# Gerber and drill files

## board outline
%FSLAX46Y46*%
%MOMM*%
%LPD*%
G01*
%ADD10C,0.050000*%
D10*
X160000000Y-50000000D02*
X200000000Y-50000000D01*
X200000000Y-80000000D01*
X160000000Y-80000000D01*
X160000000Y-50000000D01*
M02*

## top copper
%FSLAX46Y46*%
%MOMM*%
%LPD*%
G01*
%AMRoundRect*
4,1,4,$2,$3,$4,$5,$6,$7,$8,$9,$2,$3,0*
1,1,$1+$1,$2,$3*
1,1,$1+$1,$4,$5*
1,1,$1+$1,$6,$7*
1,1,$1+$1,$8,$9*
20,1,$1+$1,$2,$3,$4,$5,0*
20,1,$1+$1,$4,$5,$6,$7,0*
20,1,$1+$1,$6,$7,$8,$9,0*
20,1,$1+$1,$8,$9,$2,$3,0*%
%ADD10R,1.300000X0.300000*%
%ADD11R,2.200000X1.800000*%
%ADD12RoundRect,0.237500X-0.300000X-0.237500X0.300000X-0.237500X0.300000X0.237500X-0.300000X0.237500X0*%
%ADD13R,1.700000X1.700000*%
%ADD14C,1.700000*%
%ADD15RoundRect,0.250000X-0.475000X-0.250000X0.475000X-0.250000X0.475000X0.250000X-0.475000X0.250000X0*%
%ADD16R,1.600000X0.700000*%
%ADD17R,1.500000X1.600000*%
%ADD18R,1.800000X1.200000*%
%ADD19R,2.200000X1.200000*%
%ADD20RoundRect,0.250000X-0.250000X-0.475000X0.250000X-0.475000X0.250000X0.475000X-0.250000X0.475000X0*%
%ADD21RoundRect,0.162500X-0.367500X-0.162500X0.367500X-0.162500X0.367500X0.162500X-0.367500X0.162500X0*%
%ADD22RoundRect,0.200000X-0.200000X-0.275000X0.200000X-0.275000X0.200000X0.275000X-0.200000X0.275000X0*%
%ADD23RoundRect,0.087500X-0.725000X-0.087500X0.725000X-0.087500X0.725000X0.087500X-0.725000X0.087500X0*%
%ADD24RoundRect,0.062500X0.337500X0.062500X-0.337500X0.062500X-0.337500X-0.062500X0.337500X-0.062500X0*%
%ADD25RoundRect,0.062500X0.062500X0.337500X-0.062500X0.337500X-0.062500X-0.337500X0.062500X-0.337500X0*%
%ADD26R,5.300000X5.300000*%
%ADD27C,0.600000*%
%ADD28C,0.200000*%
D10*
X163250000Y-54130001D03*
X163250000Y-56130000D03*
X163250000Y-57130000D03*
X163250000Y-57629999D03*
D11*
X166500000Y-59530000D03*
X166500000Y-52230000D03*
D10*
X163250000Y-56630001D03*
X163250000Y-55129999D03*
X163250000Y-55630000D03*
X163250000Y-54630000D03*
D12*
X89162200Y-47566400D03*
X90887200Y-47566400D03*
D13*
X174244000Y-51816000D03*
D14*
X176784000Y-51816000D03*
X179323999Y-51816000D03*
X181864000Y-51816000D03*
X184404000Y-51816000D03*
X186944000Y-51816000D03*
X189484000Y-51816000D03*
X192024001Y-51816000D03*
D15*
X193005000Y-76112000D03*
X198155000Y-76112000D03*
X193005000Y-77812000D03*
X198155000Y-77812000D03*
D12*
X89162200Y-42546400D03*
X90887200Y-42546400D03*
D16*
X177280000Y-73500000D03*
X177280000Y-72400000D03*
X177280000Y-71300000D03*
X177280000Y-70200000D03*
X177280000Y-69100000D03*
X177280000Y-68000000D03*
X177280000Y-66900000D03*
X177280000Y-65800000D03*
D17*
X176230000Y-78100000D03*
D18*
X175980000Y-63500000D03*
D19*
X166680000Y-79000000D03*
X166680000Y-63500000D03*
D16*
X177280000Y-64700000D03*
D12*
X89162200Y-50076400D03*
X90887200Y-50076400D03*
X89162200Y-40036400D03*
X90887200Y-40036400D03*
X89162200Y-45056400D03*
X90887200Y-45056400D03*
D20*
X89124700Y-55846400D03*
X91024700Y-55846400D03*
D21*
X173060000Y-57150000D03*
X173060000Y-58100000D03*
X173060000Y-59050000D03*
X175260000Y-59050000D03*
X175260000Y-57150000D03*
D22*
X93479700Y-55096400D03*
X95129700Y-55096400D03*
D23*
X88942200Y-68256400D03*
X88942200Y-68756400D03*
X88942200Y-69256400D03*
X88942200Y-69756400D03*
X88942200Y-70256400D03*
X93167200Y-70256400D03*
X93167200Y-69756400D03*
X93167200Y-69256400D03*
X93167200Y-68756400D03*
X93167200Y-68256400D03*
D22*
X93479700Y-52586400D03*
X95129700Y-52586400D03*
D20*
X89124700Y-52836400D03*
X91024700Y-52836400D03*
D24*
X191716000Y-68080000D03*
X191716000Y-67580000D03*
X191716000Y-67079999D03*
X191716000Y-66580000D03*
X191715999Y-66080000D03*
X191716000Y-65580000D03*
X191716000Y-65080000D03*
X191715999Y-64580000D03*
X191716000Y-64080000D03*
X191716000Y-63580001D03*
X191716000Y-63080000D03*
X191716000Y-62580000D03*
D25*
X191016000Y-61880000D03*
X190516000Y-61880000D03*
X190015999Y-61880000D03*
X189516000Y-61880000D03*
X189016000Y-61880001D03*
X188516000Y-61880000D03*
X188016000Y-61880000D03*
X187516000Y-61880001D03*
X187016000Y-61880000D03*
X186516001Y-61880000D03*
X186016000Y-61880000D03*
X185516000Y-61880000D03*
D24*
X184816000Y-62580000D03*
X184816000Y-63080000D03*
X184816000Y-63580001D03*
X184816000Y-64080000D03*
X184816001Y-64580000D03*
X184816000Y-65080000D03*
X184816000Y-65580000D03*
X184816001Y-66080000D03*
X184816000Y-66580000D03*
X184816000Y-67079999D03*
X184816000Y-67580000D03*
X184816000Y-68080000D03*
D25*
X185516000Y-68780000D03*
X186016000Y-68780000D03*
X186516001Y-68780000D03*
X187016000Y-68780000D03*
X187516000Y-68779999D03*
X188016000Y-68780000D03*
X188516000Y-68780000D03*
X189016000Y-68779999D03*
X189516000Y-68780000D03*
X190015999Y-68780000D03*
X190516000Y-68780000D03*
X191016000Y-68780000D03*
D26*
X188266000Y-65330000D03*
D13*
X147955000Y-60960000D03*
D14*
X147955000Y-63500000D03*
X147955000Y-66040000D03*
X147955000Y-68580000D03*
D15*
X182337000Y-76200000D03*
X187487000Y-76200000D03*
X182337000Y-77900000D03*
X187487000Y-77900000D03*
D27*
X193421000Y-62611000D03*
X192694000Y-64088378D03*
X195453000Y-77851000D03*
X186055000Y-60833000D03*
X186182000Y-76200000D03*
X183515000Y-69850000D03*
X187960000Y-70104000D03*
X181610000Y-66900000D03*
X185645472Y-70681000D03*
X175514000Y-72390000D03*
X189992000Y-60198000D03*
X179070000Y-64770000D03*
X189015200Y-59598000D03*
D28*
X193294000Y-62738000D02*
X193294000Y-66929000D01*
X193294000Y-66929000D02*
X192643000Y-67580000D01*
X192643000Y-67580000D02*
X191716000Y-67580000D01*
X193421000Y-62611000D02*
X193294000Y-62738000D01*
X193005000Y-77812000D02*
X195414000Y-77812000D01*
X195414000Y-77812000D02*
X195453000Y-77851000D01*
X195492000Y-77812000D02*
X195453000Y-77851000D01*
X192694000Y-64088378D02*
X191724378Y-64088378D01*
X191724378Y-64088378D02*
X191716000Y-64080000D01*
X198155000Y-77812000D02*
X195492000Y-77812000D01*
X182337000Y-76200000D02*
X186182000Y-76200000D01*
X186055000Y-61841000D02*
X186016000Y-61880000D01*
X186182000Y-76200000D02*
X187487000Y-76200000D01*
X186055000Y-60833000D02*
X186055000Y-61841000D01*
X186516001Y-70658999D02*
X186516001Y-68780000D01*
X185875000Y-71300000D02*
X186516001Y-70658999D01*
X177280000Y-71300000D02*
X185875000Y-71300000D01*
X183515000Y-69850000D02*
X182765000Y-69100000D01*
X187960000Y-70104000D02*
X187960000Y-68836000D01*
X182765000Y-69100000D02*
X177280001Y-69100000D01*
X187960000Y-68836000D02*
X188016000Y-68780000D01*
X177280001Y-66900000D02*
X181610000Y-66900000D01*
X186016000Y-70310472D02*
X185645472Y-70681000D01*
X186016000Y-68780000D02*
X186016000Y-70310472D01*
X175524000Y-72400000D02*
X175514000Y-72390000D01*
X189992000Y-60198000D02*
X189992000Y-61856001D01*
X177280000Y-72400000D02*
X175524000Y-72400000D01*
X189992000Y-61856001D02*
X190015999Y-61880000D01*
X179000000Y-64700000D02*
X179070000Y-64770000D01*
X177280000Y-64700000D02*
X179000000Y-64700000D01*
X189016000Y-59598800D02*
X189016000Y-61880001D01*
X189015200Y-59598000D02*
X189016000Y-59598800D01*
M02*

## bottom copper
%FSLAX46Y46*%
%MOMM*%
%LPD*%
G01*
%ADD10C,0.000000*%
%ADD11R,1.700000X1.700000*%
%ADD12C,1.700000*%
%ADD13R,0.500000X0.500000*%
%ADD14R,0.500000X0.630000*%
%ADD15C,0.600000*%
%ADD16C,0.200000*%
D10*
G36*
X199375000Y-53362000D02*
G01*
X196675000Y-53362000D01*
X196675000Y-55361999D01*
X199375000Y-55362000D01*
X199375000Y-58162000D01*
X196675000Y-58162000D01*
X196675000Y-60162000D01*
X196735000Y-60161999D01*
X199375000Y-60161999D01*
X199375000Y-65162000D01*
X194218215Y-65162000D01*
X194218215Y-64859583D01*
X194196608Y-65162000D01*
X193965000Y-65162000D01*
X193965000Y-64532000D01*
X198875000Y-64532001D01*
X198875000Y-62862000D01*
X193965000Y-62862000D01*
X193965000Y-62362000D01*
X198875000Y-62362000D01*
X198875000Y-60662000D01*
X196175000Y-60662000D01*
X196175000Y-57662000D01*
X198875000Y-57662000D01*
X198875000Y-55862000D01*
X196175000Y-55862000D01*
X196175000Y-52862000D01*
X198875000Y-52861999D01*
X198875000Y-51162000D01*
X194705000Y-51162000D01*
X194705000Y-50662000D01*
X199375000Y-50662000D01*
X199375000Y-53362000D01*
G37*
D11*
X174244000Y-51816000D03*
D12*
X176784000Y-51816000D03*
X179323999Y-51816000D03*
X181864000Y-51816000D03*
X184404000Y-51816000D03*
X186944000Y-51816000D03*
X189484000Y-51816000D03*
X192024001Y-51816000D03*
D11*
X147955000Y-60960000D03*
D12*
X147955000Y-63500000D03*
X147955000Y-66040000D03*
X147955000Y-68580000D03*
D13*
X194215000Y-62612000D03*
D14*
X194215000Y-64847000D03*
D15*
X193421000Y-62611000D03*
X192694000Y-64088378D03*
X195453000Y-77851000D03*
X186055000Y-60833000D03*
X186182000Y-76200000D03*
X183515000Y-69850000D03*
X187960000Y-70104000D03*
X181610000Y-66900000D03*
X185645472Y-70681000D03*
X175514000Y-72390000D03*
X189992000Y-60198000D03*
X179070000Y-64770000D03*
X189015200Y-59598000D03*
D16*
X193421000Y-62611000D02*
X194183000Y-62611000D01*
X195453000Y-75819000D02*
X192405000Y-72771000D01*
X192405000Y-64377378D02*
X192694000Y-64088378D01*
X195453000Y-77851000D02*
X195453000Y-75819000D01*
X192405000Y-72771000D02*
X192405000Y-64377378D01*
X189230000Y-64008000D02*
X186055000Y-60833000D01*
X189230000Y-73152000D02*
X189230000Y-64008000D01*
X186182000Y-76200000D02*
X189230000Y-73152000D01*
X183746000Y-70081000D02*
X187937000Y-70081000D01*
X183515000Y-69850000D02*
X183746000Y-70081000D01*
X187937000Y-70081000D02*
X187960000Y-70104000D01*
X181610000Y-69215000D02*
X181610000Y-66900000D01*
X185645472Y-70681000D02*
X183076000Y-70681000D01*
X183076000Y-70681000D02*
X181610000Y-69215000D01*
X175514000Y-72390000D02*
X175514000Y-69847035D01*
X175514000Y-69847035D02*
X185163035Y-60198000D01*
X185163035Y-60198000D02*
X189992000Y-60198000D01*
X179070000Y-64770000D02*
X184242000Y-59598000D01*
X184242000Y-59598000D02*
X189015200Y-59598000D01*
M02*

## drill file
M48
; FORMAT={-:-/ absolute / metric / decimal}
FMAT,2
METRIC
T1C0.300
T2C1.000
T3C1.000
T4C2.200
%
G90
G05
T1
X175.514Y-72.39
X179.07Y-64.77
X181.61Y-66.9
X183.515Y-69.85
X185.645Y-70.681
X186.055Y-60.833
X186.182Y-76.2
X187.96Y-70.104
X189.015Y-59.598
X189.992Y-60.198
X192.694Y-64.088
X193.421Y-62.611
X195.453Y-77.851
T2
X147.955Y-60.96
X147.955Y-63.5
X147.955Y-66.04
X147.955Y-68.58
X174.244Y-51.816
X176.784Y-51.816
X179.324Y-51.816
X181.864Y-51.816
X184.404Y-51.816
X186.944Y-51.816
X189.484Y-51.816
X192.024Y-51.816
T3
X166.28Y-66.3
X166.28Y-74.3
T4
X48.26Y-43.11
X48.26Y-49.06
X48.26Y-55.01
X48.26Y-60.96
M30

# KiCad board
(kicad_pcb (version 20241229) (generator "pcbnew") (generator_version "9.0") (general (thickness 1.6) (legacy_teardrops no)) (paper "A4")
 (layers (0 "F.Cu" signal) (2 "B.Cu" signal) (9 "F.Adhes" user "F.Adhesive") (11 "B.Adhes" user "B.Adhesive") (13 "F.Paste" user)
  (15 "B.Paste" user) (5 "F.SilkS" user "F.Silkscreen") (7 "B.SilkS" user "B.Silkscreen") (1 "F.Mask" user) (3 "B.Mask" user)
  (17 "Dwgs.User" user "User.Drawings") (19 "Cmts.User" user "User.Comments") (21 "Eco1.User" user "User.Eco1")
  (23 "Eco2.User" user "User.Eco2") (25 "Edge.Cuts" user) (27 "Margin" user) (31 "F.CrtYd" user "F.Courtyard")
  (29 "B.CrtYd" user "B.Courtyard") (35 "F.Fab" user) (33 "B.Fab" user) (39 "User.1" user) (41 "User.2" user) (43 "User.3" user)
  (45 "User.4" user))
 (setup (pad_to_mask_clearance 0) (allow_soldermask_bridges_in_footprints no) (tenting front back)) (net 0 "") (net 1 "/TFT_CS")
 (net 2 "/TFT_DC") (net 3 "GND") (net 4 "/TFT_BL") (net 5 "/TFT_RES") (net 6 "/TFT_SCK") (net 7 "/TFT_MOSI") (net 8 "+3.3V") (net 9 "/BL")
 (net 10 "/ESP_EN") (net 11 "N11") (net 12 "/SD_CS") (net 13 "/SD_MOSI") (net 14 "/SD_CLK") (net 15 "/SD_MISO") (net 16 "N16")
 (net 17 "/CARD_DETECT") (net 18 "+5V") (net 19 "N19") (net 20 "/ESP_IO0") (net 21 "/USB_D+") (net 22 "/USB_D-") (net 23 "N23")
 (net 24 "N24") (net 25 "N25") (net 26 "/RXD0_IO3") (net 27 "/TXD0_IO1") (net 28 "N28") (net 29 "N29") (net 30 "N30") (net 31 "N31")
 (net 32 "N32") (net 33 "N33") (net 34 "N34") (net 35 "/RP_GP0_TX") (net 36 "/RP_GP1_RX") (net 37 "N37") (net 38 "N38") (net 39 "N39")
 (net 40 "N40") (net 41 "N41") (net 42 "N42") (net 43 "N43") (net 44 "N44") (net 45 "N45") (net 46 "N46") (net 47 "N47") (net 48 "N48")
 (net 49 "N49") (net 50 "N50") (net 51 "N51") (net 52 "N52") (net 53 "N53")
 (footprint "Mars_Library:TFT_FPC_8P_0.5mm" (layer "F.Cu") (at 165.1 55.88 90)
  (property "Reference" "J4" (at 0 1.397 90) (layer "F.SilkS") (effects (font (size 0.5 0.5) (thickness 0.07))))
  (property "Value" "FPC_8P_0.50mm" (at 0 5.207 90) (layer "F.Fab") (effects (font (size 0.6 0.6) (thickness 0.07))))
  (pad "CS" smd rect (at 1.749999 -1.85 90) (size 0.3 1.3) (layers "F.Cu" "F.Mask" "F.Paste") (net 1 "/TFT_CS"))
  (pad "DC" smd rect (at -0.25 -1.85 90) (size 0.3 1.3) (layers "F.Cu" "F.Mask" "F.Paste") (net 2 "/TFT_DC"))
  (pad "GND" smd rect (at -1.25 -1.85 90) (size 0.3 1.3) (layers "F.Cu" "F.Mask" "F.Paste") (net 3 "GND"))
  (pad "LEDA" smd rect (at -1.749999 -1.85 90) (size 0.3 1.3) (layers "F.Cu" "F.Mask" "F.Paste") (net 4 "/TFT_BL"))
  (pad "MP" smd rect (at -3.65 1.4 90) (size 1.8 2.2) (layers "F.Cu" "F.Mask" "F.Paste"))
  (pad "MP" smd rect (at 3.65 1.4 90) (size 1.8 2.2) (layers "F.Cu" "F.Mask" "F.Paste"))
  (pad "RES" smd rect (at -0.750001 -1.85 90) (size 0.3 1.3) (layers "F.Cu" "F.Mask" "F.Paste") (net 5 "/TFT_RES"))
  (pad "SCL" smd rect (at 0.750001 -1.85 90) (size 0.3 1.3) (layers "F.Cu" "F.Mask" "F.Paste") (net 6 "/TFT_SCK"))
  (pad "SDA" smd rect (at 0.25 -1.85 90) (size 0.3 1.3) (layers "F.Cu" "F.Mask" "F.Paste") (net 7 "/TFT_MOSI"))
  (pad "VDD" smd rect (at 1.25 -1.85 90) (size 0.3 1.3) (layers "F.Cu" "F.Mask" "F.Paste") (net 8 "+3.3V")))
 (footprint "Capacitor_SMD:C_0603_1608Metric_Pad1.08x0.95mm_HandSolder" (layer "F.Cu") (at 90.0247 47.5664)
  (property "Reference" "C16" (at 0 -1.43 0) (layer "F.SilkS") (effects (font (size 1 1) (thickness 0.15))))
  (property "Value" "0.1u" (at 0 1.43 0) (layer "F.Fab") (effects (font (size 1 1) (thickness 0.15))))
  (pad "1" smd roundrect (at -0.8625 0) (size 1.075 0.95) (layers "F.Cu" "F.Mask" "F.Paste") (roundrect_rratio 0.25) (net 8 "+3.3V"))
  (pad "2" smd roundrect (at 0.8625 0) (size 1.075 0.95) (layers "F.Cu" "F.Mask" "F.Paste") (roundrect_rratio 0.25) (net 3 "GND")))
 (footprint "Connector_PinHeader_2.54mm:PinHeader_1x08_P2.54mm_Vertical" (layer "F.Cu") (at 174.244 51.816 90)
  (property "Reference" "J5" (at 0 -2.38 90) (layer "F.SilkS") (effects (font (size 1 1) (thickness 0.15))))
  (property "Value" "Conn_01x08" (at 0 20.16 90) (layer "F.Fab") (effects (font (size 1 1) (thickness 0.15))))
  (pad "1" thru_hole rect (at 0 0 90) (size 1.7 1.7) (drill 1) (layers "*.Cu" "*.Mask") (remove_unused_layers no) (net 3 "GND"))
  (pad "2" thru_hole circle (at 0 2.54 90) (size 1.7 1.7) (drill 1) (layers "*.Cu" "*.Mask") (remove_unused_layers no) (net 8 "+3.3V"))
  (pad "3" thru_hole circle (at 0 5.079999 90) (size 1.7 1.7) (drill 1) (layers "*.Cu" "*.Mask") (remove_unused_layers no)
   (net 6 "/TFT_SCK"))
  (pad "4" thru_hole circle (at 0 7.62 90) (size 1.7 1.7) (drill 1) (layers "*.Cu" "*.Mask") (remove_unused_layers no) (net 7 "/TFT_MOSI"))
  (pad "5" thru_hole circle (at 0 10.16 90) (size 1.7 1.7) (drill 1) (layers "*.Cu" "*.Mask") (remove_unused_layers no) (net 5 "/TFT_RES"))
  (pad "6" thru_hole circle (at 0 12.7 90) (size 1.7 1.7) (drill 1) (layers "*.Cu" "*.Mask") (remove_unused_layers no) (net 2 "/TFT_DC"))
  (pad "7" thru_hole circle (at 0 15.24 90) (size 1.7 1.7) (drill 1) (layers "*.Cu" "*.Mask") (remove_unused_layers no) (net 1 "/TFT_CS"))
  (pad "8" thru_hole circle (at 0 17.780001 90) (size 1.7 1.7) (drill 1) (layers "*.Cu" "*.Mask") (remove_unused_layers no) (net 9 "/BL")))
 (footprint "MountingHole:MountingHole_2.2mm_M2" (layer "F.Cu") (at 48.26 49.06)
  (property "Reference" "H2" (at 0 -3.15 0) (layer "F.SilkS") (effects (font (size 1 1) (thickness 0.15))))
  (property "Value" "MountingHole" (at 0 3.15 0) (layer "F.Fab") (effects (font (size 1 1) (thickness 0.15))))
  (pad "" np_thru_hole circle (at 0 0) (size 2.2 2.2) (drill 2.2) (layers "*.Cu" "*.Mask")))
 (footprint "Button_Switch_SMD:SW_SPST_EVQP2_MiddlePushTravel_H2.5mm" (layer "F.Cu") (at 195.58 76.962)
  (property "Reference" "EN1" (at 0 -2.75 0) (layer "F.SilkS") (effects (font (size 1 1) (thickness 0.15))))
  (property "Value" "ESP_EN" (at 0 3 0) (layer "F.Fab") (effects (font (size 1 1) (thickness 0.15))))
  (pad "1" smd roundrect (at -2.575 -0.85) (size 1.45 1) (layers "F.Cu" "F.Mask" "F.Paste") (roundrect_rratio 0.25) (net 3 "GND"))
  (pad "1" smd roundrect (at 2.575 -0.85) (size 1.45 1) (layers "F.Cu" "F.Mask" "F.Paste") (roundrect_rratio 0.25) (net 3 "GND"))
  (pad "2" smd roundrect (at -2.575 0.85) (size 1.45 1) (layers "F.Cu" "F.Mask" "F.Paste") (roundrect_rratio 0.25) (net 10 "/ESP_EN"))
  (pad "2" smd roundrect (at 2.575 0.85) (size 1.45 1) (layers "F.Cu" "F.Mask" "F.Paste") (roundrect_rratio 0.25) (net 10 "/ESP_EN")))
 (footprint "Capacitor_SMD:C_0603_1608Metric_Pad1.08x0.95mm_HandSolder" (layer "F.Cu") (at 90.0247 42.5464)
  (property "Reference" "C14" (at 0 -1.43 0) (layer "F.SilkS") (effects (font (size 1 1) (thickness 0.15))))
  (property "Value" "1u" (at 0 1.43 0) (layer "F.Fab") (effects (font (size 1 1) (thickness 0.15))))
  (pad "1" smd roundrect (at -0.8625 0) (size 1.075 0.95) (layers "F.Cu" "F.Mask" "F.Paste") (roundrect_rratio 0.25) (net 8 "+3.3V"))
  (pad "2" smd roundrect (at 0.8625 0) (size 1.075 0.95) (layers "F.Cu" "F.Mask" "F.Paste") (roundrect_rratio 0.25) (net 3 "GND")))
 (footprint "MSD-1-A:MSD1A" (layer "F.Cu") (at 170.18 71.25 -90)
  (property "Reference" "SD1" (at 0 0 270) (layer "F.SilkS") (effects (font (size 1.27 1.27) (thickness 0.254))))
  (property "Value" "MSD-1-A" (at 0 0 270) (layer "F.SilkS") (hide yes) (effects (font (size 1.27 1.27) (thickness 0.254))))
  (pad "" np_thru_hole circle (at -4.95 3.9 270) (size 1 1) (drill 1) (layers "*.Cu" "*.Mask"))
  (pad "" np_thru_hole circle (at 3.05 3.9 270) (size 1 1) (drill 1) (layers "*.Cu" "*.Mask"))
  (pad "1" smd rect (at 2.25 -7.1 270) (size 0.7 1.6) (layers "F.Cu" "F.Mask" "F.Paste") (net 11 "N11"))
  (pad "2" smd rect (at 1.15 -7.1 270) (size 0.7 1.6) (layers "F.Cu" "F.Mask" "F.Paste") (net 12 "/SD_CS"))
  (pad "3" smd rect (at 0.05 -7.1 270) (size 0.7 1.6) (layers "F.Cu" "F.Mask" "F.Paste") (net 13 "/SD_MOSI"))
  (pad "4" smd rect (at -1.05 -7.1 270) (size 0.7 1.6) (layers "F.Cu" "F.Mask" "F.Paste") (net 8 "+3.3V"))
  (pad "5" smd rect (at -2.15 -7.1 270) (size 0.7 1.6) (layers "F.Cu" "F.Mask" "F.Paste") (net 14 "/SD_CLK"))
  (pad "6" smd rect (at -3.25 -7.1 270) (size 0.7 1.6) (layers "F.Cu" "F.Mask" "F.Paste") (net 3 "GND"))
  (pad "7" smd rect (at -4.35 -7.1 270) (size 0.7 1.6) (layers "F.Cu" "F.Mask" "F.Paste") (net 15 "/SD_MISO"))
  (pad "8" smd rect (at -5.45 -7.1 270) (size 0.7 1.6) (layers "F.Cu" "F.Mask" "F.Paste") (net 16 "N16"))
  (pad "9" smd rect (at 6.85 -6.05) (size 1.5 1.6) (layers "F.Cu" "F.Mask" "F.Paste") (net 3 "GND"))
  (pad "10" smd rect (at -7.75 -5.8 270) (size 1.2 1.8) (layers "F.Cu" "F.Mask" "F.Paste") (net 3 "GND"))
  (pad "11" smd rect (at 7.75 3.5 270) (size 1.2 2.2) (layers "F.Cu" "F.Mask" "F.Paste") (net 3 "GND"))
  (pad "12" smd rect (at -7.75 3.5 270) (size 1.2 2.2) (layers "F.Cu" "F.Mask" "F.Paste") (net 3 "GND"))
  (pad "CD1" smd rect (at -6.55 -7.1 270) (size 0.7 1.6) (layers "F.Cu" "F.Mask" "F.Paste") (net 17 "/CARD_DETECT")))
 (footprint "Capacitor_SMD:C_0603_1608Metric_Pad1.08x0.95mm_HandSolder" (layer "F.Cu") (at 90.0247 50.0764)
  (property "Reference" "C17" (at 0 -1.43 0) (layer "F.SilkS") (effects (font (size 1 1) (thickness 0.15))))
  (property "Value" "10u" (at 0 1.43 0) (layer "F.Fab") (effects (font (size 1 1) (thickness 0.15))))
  (pad "1" smd roundrect (at -0.8625 0) (size 1.075 0.95) (layers "F.Cu" "F.Mask" "F.Paste") (roundrect_rratio 0.25) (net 8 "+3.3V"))
  (pad "2" smd roundrect (at 0.8625 0) (size 1.075 0.95) (layers "F.Cu" "F.Mask" "F.Paste") (roundrect_rratio 0.25) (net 3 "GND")))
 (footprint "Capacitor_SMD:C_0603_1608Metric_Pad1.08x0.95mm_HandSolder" (layer "F.Cu") (at 90.0247 40.0364)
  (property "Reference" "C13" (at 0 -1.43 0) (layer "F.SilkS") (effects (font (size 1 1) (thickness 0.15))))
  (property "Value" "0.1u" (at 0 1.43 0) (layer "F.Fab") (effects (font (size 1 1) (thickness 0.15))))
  (pad "1" smd roundrect (at -0.8625 0) (size 1.075 0.95) (layers "F.Cu" "F.Mask" "F.Paste") (roundrect_rratio 0.25) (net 8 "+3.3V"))
  (pad "2" smd roundrect (at 0.8625 0) (size 1.075 0.95) (layers "F.Cu" "F.Mask" "F.Paste") (roundrect_rratio 0.25) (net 3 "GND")))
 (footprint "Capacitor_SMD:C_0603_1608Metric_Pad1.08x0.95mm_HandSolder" (layer "F.Cu") (at 90.0247 45.0564)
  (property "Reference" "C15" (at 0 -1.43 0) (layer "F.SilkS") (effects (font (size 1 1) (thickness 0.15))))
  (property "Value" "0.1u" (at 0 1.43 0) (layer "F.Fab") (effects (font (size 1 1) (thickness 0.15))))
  (pad "1" smd roundrect (at -0.8625 0) (size 1.075 0.95) (layers "F.Cu" "F.Mask" "F.Paste") (roundrect_rratio 0.25) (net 8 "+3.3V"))
  (pad "2" smd roundrect (at 0.8625 0) (size 1.075 0.95) (layers "F.Cu" "F.Mask" "F.Paste") (roundrect_rratio 0.25) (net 3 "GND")))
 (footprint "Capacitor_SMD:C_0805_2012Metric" (layer "F.Cu") (at 90.0747 55.8464)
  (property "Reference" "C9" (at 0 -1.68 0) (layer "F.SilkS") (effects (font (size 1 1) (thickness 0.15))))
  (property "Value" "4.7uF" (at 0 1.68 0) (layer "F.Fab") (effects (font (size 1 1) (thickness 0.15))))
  (pad "1" smd roundrect (at -0.95 0) (size 1 1.45) (layers "F.Cu" "F.Mask" "F.Paste") (roundrect_rratio 0.25) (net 8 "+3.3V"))
  (pad "2" smd roundrect (at 0.95 0) (size 1 1.45) (layers "F.Cu" "F.Mask" "F.Paste") (roundrect_rratio 0.25) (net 3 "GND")))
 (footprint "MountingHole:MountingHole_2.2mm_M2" (layer "F.Cu") (at 48.26 60.96)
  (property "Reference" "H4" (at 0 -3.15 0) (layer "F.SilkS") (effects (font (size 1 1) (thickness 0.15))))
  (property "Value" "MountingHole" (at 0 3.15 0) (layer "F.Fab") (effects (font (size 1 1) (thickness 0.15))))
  (pad "" np_thru_hole circle (at 0 0) (size 2.2 2.2) (drill 2.2) (layers "*.Cu" "*.Mask")))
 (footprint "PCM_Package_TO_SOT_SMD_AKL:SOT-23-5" (layer "F.Cu") (at 174.16 58.1)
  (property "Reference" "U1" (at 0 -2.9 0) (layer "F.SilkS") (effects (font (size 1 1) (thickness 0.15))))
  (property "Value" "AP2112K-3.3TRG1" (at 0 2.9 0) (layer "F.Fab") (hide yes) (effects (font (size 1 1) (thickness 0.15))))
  (pad "1" smd roundrect (at -1.1 -0.95) (size 1.06 0.65) (layers "F.Cu" "F.Mask" "F.Paste") (roundrect_rratio 0.25) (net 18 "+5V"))
  (pad "2" smd roundrect (at -1.1 0) (size 1.06 0.65) (layers "F.Cu" "F.Mask" "F.Paste") (roundrect_rratio 0.25) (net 3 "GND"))
  (pad "3" smd roundrect (at -1.1 0.95) (size 1.06 0.65) (layers "F.Cu" "F.Mask" "F.Paste") (roundrect_rratio 0.25) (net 18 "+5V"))
  (pad "4" smd roundrect (at 1.1 0.95) (size 1.06 0.65) (layers "F.Cu" "F.Mask" "F.Paste") (roundrect_rratio 0.25) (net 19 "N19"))
  (pad "5" smd roundrect (at 1.1 -0.95) (size 1.06 0.65) (layers "F.Cu" "F.Mask" "F.Paste") (roundrect_rratio 0.25) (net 8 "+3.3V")))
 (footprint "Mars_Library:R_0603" (layer "F.Cu") (at 94.3047 55.0964)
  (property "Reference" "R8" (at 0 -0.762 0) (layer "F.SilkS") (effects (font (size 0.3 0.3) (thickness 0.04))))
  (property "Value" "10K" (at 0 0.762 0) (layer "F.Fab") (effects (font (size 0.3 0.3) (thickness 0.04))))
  (pad "1" smd roundrect (at -0.825 0) (size 0.8 0.95) (layers "F.Cu" "F.Mask" "F.Paste") (roundrect_rratio 0.25) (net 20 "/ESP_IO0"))
  (pad "2" smd roundrect (at 0.825 0) (size 0.8 0.95) (layers "F.Cu" "F.Mask" "F.Paste") (roundrect_rratio 0.25) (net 8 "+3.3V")))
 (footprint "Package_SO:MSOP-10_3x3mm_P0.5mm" (layer "F.Cu") (at 91.0547 69.2564)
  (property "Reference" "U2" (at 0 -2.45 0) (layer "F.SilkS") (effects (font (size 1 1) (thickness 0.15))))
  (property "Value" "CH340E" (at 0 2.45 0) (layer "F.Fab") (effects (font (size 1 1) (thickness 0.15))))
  (pad "1" smd roundrect (at -2.1125 -1) (size 1.625 0.35) (layers "F.Cu" "F.Mask" "F.Paste") (roundrect_rratio 0.25) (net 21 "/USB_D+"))
  (pad "2" smd roundrect (at -2.1125 -0.5) (size 1.625 0.35) (layers "F.Cu" "F.Mask" "F.Paste") (roundrect_rratio 0.25) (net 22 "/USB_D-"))
  (pad "3" smd roundrect (at -2.1125 0) (size 1.625 0.35) (layers "F.Cu" "F.Mask" "F.Paste") (roundrect_rratio 0.25) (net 3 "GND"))
  (pad "4" smd roundrect (at -2.1125 0.5) (size 1.625 0.35) (layers "F.Cu" "F.Mask" "F.Paste") (roundrect_rratio 0.25) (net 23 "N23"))
  (pad "5" smd roundrect (at -2.1125 1) (size 1.625 0.35) (layers "F.Cu" "F.Mask" "F.Paste") (roundrect_rratio 0.25) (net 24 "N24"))
  (pad "6" smd roundrect (at 2.1125 1) (size 1.625 0.35) (layers "F.Cu" "F.Mask" "F.Paste") (roundrect_rratio 0.25) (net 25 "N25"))
  (pad "7" smd roundrect (at 2.1125 0.5) (size 1.625 0.35) (layers "F.Cu" "F.Mask" "F.Paste") (roundrect_rratio 0.25) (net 8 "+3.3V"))
  (pad "8" smd roundrect (at 2.1125 0) (size 1.625 0.35) (layers "F.Cu" "F.Mask" "F.Paste") (roundrect_rratio 0.25) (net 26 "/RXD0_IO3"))
  (pad "9" smd roundrect (at 2.1125 -0.5) (size 1.625 0.35) (layers "F.Cu" "F.Mask" "F.Paste") (roundrect_rratio 0.25) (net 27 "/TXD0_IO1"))
  (pad "10" smd roundrect (at 2.1125 -1) (size 1.625 0.35) (layers "F.Cu" "F.Mask" "F.Paste") (roundrect_rratio 0.25) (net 8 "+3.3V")))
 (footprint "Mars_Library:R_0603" (layer "F.Cu") (at 94.3047 52.5864)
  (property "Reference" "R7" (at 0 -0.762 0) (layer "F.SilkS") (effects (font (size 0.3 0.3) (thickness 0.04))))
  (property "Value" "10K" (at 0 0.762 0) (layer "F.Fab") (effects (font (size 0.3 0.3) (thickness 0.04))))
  (pad "1" smd roundrect (at -0.825 0) (size 0.8 0.95) (layers "F.Cu" "F.Mask" "F.Paste") (roundrect_rratio 0.25) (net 10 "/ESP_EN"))
  (pad "2" smd roundrect (at 0.825 0) (size 0.8 0.95) (layers "F.Cu" "F.Mask" "F.Paste") (roundrect_rratio 0.25) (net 8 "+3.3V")))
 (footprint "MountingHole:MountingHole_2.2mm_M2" (layer "F.Cu") (at 48.26 43.11)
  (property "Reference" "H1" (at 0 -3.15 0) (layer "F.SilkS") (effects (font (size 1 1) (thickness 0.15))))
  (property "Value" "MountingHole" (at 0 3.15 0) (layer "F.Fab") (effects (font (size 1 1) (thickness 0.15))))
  (pad "" np_thru_hole circle (at 0 0) (size 2.2 2.2) (drill 2.2) (layers "*.Cu" "*.Mask")))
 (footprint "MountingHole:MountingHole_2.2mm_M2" (layer "F.Cu") (at 48.26 55.01)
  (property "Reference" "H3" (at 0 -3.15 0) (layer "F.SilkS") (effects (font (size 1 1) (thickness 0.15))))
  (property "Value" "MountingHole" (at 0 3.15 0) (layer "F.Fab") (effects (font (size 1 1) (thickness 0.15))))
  (pad "" np_thru_hole circle (at 0 0) (size 2.2 2.2) (drill 2.2) (layers "*.Cu" "*.Mask")))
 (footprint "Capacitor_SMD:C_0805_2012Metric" (layer "F.Cu") (at 90.0747 52.8364)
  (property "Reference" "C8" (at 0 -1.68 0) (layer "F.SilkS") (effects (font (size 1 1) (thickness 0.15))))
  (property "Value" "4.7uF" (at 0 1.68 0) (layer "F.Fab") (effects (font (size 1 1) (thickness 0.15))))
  (pad "1" smd roundrect (at -0.95 0) (size 1 1.45) (layers "F.Cu" "F.Mask" "F.Paste") (roundrect_rratio 0.25) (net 18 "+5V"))
  (pad "2" smd roundrect (at 0.95 0) (size 1 1.45) (layers "F.Cu" "F.Mask" "F.Paste") (roundrect_rratio 0.25) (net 3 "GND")))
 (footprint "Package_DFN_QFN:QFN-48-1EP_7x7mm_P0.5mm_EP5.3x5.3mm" (layer "F.Cu") (at 188.266 65.33 180)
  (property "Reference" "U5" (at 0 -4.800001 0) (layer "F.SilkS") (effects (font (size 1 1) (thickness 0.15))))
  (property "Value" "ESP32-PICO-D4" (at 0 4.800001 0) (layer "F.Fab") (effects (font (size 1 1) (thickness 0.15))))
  (pad "" smd roundrect (at -1.98 -1.98 180) (size 1.07 1.07) (layers "F.Paste") (roundrect_rratio 0.233645))
  (pad "" smd roundrect (at -1.98 -0.66 180) (size 1.07 1.07) (layers "F.Paste") (roundrect_rratio 0.233645))
  (pad "" smd roundrect (at -1.98 0.66 180) (size 1.07 1.07) (layers "F.Paste") (roundrect_rratio 0.233645))
  (pad "" smd roundrect (at -1.98 1.98 180) (size 1.07 1.07) (layers "F.Paste") (roundrect_rratio 0.233645))
  (pad "" smd roundrect (at -0.66 -1.98 180) (size 1.07 1.07) (layers "F.Paste") (roundrect_rratio 0.233645))
  (pad "" smd roundrect (at -0.66 -0.66 180) (size 1.07 1.07) (layers "F.Paste") (roundrect_rratio 0.233645))
  (pad "" smd roundrect (at -0.66 0.66 180) (size 1.07 1.07) (layers "F.Paste") (roundrect_rratio 0.233645))
  (pad "" smd roundrect (at -0.66 1.98 180) (size 1.07 1.07) (layers "F.Paste") (roundrect_rratio 0.233645))
  (pad "" smd roundrect (at 0.66 -1.98 180) (size 1.07 1.07) (layers "F.Paste") (roundrect_rratio 0.233645))
  (pad "" smd roundrect (at 0.66 -0.66 180) (size 1.07 1.07) (layers "F.Paste") (roundrect_rratio 0.233645))
  (pad "" smd roundrect (at 0.66 0.66 180) (size 1.07 1.07) (layers "F.Paste") (roundrect_rratio 0.233645))
  (pad "" smd roundrect (at 0.66 1.98 180) (size 1.07 1.07) (layers "F.Paste") (roundrect_rratio 0.233645))
  (pad "" smd roundrect (at 1.98 -1.98 180) (size 1.07 1.07) (layers "F.Paste") (roundrect_rratio 0.233645))
  (pad "" smd roundrect (at 1.98 -0.66 180) (size 1.07 1.07) (layers "F.Paste") (roundrect_rratio 0.233645))
  (pad "" smd roundrect (at 1.98 0.66 180) (size 1.07 1.07) (layers "F.Paste") (roundrect_rratio 0.233645))
  (pad "" smd roundrect (at 1.98 1.98 180) (size 1.07 1.07) (layers "F.Paste") (roundrect_rratio 0.233645))
  (pad "1" smd roundrect (at -3.45 -2.75 180) (size 0.8 0.25) (layers "F.Cu" "F.Mask" "F.Paste") (roundrect_rratio 0.25) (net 8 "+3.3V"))
  (pad "2" smd roundrect (at -3.45 -2.25 180) (size 0.8 0.25) (layers "F.Cu" "F.Mask" "F.Paste") (roundrect_rratio 0.25) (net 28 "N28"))
  (pad "3" smd roundrect (at -3.45 -1.749999 180) (size 0.8 0.25) (layers "F.Cu" "F.Mask" "F.Paste") (roundrect_rratio 0.25) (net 8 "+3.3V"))
  (pad "4" smd roundrect (at -3.45 -1.25 180) (size 0.8 0.25) (layers "F.Cu" "F.Mask" "F.Paste") (roundrect_rratio 0.25) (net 8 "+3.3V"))
  (pad "5" smd roundrect (at -3.449999 -0.75 180) (size 0.8 0.25) (layers "F.Cu" "F.Mask" "F.Paste") (roundrect_rratio 0.25) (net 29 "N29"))
  (pad "6" smd roundrect (at -3.45 -0.25 180) (size 0.8 0.25) (layers "F.Cu" "F.Mask" "F.Paste") (roundrect_rratio 0.25) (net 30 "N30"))
  (pad "7" smd roundrect (at -3.45 0.25 180) (size 0.8 0.25) (layers "F.Cu" "F.Mask" "F.Paste") (roundrect_rratio 0.25) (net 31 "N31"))
  (pad "8" smd roundrect (at -3.449999 0.75 180) (size 0.8 0.25) (layers "F.Cu" "F.Mask" "F.Paste") (roundrect_rratio 0.25) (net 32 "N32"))
  (pad "9" smd roundrect (at -3.45 1.25 180) (size 0.8 0.25) (layers "F.Cu" "F.Mask" "F.Paste") (roundrect_rratio 0.25) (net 10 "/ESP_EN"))
  (pad "10" smd roundrect (at -3.45 1.749999 180) (size 0.8 0.25) (layers "F.Cu" "F.Mask" "F.Paste") (roundrect_rratio 0.25) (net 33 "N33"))
  (pad "11" smd roundrect (at -3.45 2.25 180) (size 0.8 0.25) (layers "F.Cu" "F.Mask" "F.Paste") (roundrect_rratio 0.25) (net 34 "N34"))
  (pad "12" smd roundrect (at -3.45 2.75 180) (size 0.8 0.25) (layers "F.Cu" "F.Mask" "F.Paste") (roundrect_rratio 0.25)
   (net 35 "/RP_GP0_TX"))
  (pad "13" smd roundrect (at -2.75 3.45 180) (size 0.25 0.8) (layers "F.Cu" "F.Mask" "F.Paste") (roundrect_rratio 0.25)
   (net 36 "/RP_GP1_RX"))
  (pad "14" smd roundrect (at -2.25 3.45 180) (size 0.25 0.8) (layers "F.Cu" "F.Mask" "F.Paste") (roundrect_rratio 0.25) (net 4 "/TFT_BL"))
  (pad "15" smd roundrect (at -1.749999 3.45 180) (size 0.25 0.8) (layers "F.Cu" "F.Mask" "F.Paste") (roundrect_rratio 0.25)
   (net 12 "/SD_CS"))
  (pad "16" smd roundrect (at -1.25 3.45 180) (size 0.25 0.8) (layers "F.Cu" "F.Mask" "F.Paste") (roundrect_rratio 0.25) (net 1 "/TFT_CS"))
  (pad "17" smd roundrect (at -0.75 3.449999 180) (size 0.25 0.8) (layers "F.Cu" "F.Mask" "F.Paste") (roundrect_rratio 0.25)
   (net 17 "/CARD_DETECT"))
  (pad "18" smd roundrect (at -0.25 3.45 180) (size 0.25 0.8) (layers "F.Cu" "F.Mask" "F.Paste") (roundrect_rratio 0.25) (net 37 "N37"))
  (pad "19" smd roundrect (at 0.25 3.45 180) (size 0.25 0.8) (layers "F.Cu" "F.Mask" "F.Paste") (roundrect_rratio 0.25) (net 8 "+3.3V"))
  (pad "20" smd roundrect (at 0.75 3.449999 180) (size 0.25 0.8) (layers "F.Cu" "F.Mask" "F.Paste") (roundrect_rratio 0.25) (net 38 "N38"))
  (pad "21" smd roundrect (at 1.25 3.45 180) (size 0.25 0.8) (layers "F.Cu" "F.Mask" "F.Paste") (roundrect_rratio 0.25) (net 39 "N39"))
  (pad "22" smd roundrect (at 1.749999 3.45 180) (size 0.25 0.8) (layers "F.Cu" "F.Mask" "F.Paste") (roundrect_rratio 0.25)
   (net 2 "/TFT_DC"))
  (pad "23" smd roundrect (at 2.25 3.45 180) (size 0.25 0.8) (layers "F.Cu" "F.Mask" "F.Paste") (roundrect_rratio 0.25) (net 20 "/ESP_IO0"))
  (pad "24" smd roundrect (at 2.75 3.45 180) (size 0.25 0.8) (layers "F.Cu" "F.Mask" "F.Paste") (roundrect_rratio 0.25) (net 5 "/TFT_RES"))
  (pad "25" smd roundrect (at 3.45 2.75 180) (size 0.8 0.25) (layers "F.Cu" "F.Mask" "F.Paste") (roundrect_rratio 0.25) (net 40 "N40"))
  (pad "26" smd roundrect (at 3.45 2.25 180) (size 0.8 0.25) (layers "F.Cu" "F.Mask" "F.Paste") (roundrect_rratio 0.25) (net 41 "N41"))
  (pad "27" smd roundrect (at 3.45 1.749999 180) (size 0.8 0.25) (layers "F.Cu" "F.Mask" "F.Paste") (roundrect_rratio 0.25) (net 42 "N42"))
  (pad "28" smd roundrect (at 3.45 1.25 180) (size 0.8 0.25) (layers "F.Cu" "F.Mask" "F.Paste") (roundrect_rratio 0.25) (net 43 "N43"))
  (pad "29" smd roundrect (at 3.449999 0.75 180) (size 0.8 0.25) (layers "F.Cu" "F.Mask" "F.Paste") (roundrect_rratio 0.25) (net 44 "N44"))
  (pad "30" smd roundrect (at 3.45 0.25 180) (size 0.8 0.25) (layers "F.Cu" "F.Mask" "F.Paste") (roundrect_rratio 0.25) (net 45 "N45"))
  (pad "31" smd roundrect (at 3.45 -0.25 180) (size 0.8 0.25) (layers "F.Cu" "F.Mask" "F.Paste") (roundrect_rratio 0.25) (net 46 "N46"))
  (pad "32" smd roundrect (at 3.449999 -0.75 180) (size 0.8 0.25) (layers "F.Cu" "F.Mask" "F.Paste") (roundrect_rratio 0.25) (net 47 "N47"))
  (pad "33" smd roundrect (at 3.45 -1.25 180) (size 0.8 0.25) (layers "F.Cu" "F.Mask" "F.Paste") (roundrect_rratio 0.25) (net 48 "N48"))
  (pad "34" smd roundrect (at 3.45 -1.749999 180) (size 0.8 0.25) (layers "F.Cu" "F.Mask" "F.Paste") (roundrect_rratio 0.25) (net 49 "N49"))
  (pad "35" smd roundrect (at 3.45 -2.25 180) (size 0.8 0.25) (layers "F.Cu" "F.Mask" "F.Paste") (roundrect_rratio 0.25) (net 6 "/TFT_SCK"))
  (pad "36" smd roundrect (at 3.45 -2.75 180) (size 0.8 0.25) (layers "F.Cu" "F.Mask" "F.Paste") (roundrect_rratio 0.25) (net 7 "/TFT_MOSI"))
  (pad "37" smd roundrect (at 2.75 -3.45 180) (size 0.25 0.8) (layers "F.Cu" "F.Mask" "F.Paste") (roundrect_rratio 0.25) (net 8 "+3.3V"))
  (pad "38" smd roundrect (at 2.25 -3.45 180) (size 0.25 0.8) (layers "F.Cu" "F.Mask" "F.Paste") (roundrect_rratio 0.25) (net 15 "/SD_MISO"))
  (pad "39" smd roundrect (at 1.749999 -3.45 180) (size 0.25 0.8) (layers "F.Cu" "F.Mask" "F.Paste") (roundrect_rratio 0.25)
   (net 13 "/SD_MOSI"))
  (pad "40" smd roundrect (at 1.25 -3.45 180) (size 0.25 0.8) (layers "F.Cu" "F.Mask" "F.Paste") (roundrect_rratio 0.25)
   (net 26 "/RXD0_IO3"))
  (pad "41" smd roundrect (at 0.75 -3.449999 180) (size 0.25 0.8) (layers "F.Cu" "F.Mask" "F.Paste") (roundrect_rratio 0.25)
   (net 27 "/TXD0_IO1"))
  (pad "42" smd roundrect (at 0.25 -3.45 180) (size 0.25 0.8) (layers "F.Cu" "F.Mask" "F.Paste") (roundrect_rratio 0.25) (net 14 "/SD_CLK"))
  (pad "43" smd roundrect (at -0.25 -3.45 180) (size 0.25 0.8) (layers "F.Cu" "F.Mask" "F.Paste") (roundrect_rratio 0.25) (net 8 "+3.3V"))
  (pad "44" smd roundrect (at -0.75 -3.449999 180) (size 0.25 0.8) (layers "F.Cu" "F.Mask" "F.Paste") (roundrect_rratio 0.25) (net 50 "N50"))
  (pad "45" smd roundrect (at -1.25 -3.45 180) (size 0.25 0.8) (layers "F.Cu" "F.Mask" "F.Paste") (roundrect_rratio 0.25) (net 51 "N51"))
  (pad "46" smd roundrect (at -1.749999 -3.45 180) (size 0.25 0.8) (layers "F.Cu" "F.Mask" "F.Paste") (roundrect_rratio 0.25)
   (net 8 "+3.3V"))
  (pad "47" smd roundrect (at -2.25 -3.45 180) (size 0.25 0.8) (layers "F.Cu" "F.Mask" "F.Paste") (roundrect_rratio 0.25) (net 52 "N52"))
  (pad "48" smd roundrect (at -2.75 -3.45 180) (size 0.25 0.8) (layers "F.Cu" "F.Mask" "F.Paste") (roundrect_rratio 0.25) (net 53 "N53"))
  (pad "49" smd rect (at 0 0 180) (size 5.3 5.3) (layers "F.Cu" "F.Mask") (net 3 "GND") (zone_connect 2)))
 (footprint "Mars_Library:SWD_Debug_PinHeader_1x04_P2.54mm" (layer "F.Cu") (at 147.955 60.96)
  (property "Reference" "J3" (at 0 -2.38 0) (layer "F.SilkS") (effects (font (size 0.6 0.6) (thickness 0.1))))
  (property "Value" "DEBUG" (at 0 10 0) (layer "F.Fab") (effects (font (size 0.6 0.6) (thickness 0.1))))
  (pad "1" thru_hole rect (at 0 0) (size 1.7 1.7) (drill 1) (layers "*.Cu" "*.Mask") (remove_unused_layers no) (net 26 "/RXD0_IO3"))
  (pad "2" thru_hole circle (at 0 2.54) (size 1.7 1.7) (drill 1) (layers "*.Cu" "*.Mask") (remove_unused_layers no) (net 27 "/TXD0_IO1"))
  (pad "3" thru_hole circle (at 0 5.08) (size 1.7 1.7) (drill 1) (layers "*.Cu" "*.Mask") (remove_unused_layers no) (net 3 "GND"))
  (pad "4" thru_hole circle (at 0 7.62) (size 1.7 1.7) (drill 1) (layers "*.Cu" "*.Mask") (remove_unused_layers no) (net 8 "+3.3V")))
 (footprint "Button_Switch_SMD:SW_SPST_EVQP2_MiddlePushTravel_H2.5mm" (layer "F.Cu") (at 184.912 77.05)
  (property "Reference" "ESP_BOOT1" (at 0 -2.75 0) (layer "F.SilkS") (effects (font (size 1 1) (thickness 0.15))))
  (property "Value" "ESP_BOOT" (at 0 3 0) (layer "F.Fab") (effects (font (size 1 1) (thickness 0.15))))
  (pad "1" smd roundrect (at -2.575 -0.85) (size 1.45 1) (layers "F.Cu" "F.Mask" "F.Paste") (roundrect_rratio 0.25) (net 20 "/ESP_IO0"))
  (pad "1" smd roundrect (at 2.575 -0.85) (size 1.45 1) (layers "F.Cu" "F.Mask" "F.Paste") (roundrect_rratio 0.25) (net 20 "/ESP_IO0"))
  (pad "2" smd roundrect (at -2.575 0.85) (size 1.45 1) (layers "F.Cu" "F.Mask" "F.Paste") (roundrect_rratio 0.25) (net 3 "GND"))
  (pad "2" smd roundrect (at 2.575 0.85) (size 1.45 1) (layers "F.Cu" "F.Mask" "F.Paste") (roundrect_rratio 0.25) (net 3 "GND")))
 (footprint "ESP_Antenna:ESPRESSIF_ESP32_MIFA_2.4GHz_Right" (layer "B.Cu") (at 194.225 62.462 90)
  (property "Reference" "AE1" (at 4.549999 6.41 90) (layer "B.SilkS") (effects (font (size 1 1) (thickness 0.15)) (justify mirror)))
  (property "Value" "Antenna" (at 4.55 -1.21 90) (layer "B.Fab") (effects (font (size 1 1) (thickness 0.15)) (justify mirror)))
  (fp_poly
   (pts (xy 2.3 2.45) (xy 4.3 2.45) (xy 4.3 5.15) (xy 7.1 5.15) (xy 7.100001 2.45) (xy 9.1 2.45) (xy 9.1 5.15) (xy 11.8 5.15) (xy 11.8 0.48)
    (xy 11.3 0.48) (xy 11.3 4.65) (xy 9.600001 4.65) (xy 9.6 1.95) (xy 6.6 1.95) (xy 6.6 4.65) (xy 4.8 4.65) (xy 4.8 1.95) (xy 1.8 1.95)
    (xy 1.8 4.65) (xy 0.1 4.65) (xy 0.1 -0.26) (xy -0.4 -0.26) (xy -0.4 4.65) (xy -2.070001 4.65) (xy -2.07 -0.26) (xy -2.7 -0.26)
    (xy -2.7 -0.006785) (xy -2.397583 -0.006785) (xy -2.387742 -0.054396) (xy -2.363674 -0.096797) (xy -2.325731 -0.129581)
    (xy -2.317819 -0.133935) (xy -2.275156 -0.146043) (xy -2.226638 -0.1453) (xy -2.181122 -0.1324) (xy -2.162511 -0.121787)
    (xy -2.128868 -0.086553) (xy -2.108309 -0.041368) (xy -2.101778 0.008158) (xy -2.110218 0.056417) (xy -2.127112 0.088643)
    (xy -2.162372 0.121313) (xy -2.207681 0.141408) (xy -2.257267 0.147982) (xy -2.305353 0.140092) (xy -2.338245 0.123186)
    (xy -2.373185 0.086416) (xy -2.392847 0.041622) (xy -2.397583 -0.006785) (xy -2.7 -0.028392) (xy -2.7 5.15) (xy 2.300001 5.15)
    (xy 2.300001 2.51))
   (stroke (width 0) (type solid)) (fill yes) (layer "B.Cu"))
  (pad "1" connect rect (at -0.15 -0.01 90) (size 0.5 0.5) (layers "B.Cu") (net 28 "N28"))
  (pad "2" smd rect (at -2.385 -0.01 90) (size 0.63 0.5) (layers "B.Cu" "B.Mask") (zone_connect 2)))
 (gr_rect (start 160 50) (end 200 80) (stroke (width 0.05) (type default)) (fill no) (layer "Edge.Cuts"))
 (segment (start 193.294 62.738) (end 193.294 66.929) (width 0.2) (layer "F.Cu") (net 28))
 (segment (start 193.294 66.929) (end 192.643 67.58) (width 0.2) (layer "F.Cu") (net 28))
 (segment (start 192.643 67.58) (end 191.716 67.58) (width 0.2) (layer "F.Cu") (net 28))
 (segment (start 193.421 62.611) (end 193.294 62.738) (width 0.2) (layer "F.Cu") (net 28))
 (via (at 193.421 62.611) (size 0.6) (drill 0.3) (layers "F.Cu" "B.Cu") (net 28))
 (segment (start 193.421 62.611) (end 194.183 62.611) (width 0.2) (layer "B.Cu") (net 28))
 (segment (start 193.005 77.812) (end 195.414 77.812) (width 0.2) (layer "F.Cu") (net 10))
 (segment (start 195.414 77.812) (end 195.453 77.851) (width 0.2) (layer "F.Cu") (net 10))
 (segment (start 195.492 77.812) (end 195.453 77.851) (width 0.2) (layer "F.Cu") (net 10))
 (segment (start 192.694 64.088378) (end 191.724378 64.088378) (width 0.2) (layer "F.Cu") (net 10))
 (segment (start 191.724378 64.088378) (end 191.716 64.08) (width 0.2) (layer "F.Cu") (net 10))
 (segment (start 198.155 77.812) (end 195.492 77.812) (width 0.2) (layer "F.Cu") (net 10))
 (via (at 192.694 64.088378) (size 0.6) (drill 0.3) (layers "F.Cu" "B.Cu") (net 10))
 (via (at 195.453 77.851) (size 0.6) (drill 0.3) (layers "F.Cu" "B.Cu") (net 10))
 (segment (start 195.453 75.819) (end 192.405 72.771) (width 0.2) (layer "B.Cu") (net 10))
 (segment (start 192.405 64.377378) (end 192.694 64.088378) (width 0.2) (layer "B.Cu") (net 10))
 (segment (start 195.453 77.851) (end 195.453 75.819) (width 0.2) (layer "B.Cu") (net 10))
 (segment (start 192.405 72.771) (end 192.405 64.377378) (width 0.2) (layer "B.Cu") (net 10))
 (segment (start 182.337 76.2) (end 186.182 76.2) (width 0.2) (layer "F.Cu") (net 20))
 (segment (start 186.055 61.841) (end 186.016 61.88) (width 0.2) (layer "F.Cu") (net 20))
 (segment (start 186.182 76.2) (end 187.487 76.2) (width 0.2) (layer "F.Cu") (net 20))
 (segment (start 186.055 60.833) (end 186.055 61.841) (width 0.2) (layer "F.Cu") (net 20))
 (via (at 186.055 60.833) (size 0.6) (drill 0.3) (layers "F.Cu" "B.Cu") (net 20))
 (via (at 186.182 76.2) (size 0.6) (drill 0.3) (layers "F.Cu" "B.Cu") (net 20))
 (segment (start 189.23 64.008) (end 186.055 60.833) (width 0.2) (layer "B.Cu") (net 20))
 (segment (start 189.23 73.152) (end 189.23 64.008) (width 0.2) (layer "B.Cu") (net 20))
 (segment (start 186.182 76.2) (end 189.23 73.152) (width 0.2) (layer "B.Cu") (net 20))
 (segment (start 186.516001 70.658999) (end 186.516001 68.78) (width 0.2) (layer "F.Cu") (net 13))
 (segment (start 185.875 71.3) (end 186.516001 70.658999) (width 0.2) (layer "F.Cu") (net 13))
 (segment (start 177.28 71.3) (end 185.875 71.3) (width 0.2) (layer "F.Cu") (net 13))
 (segment (start 183.515 69.85) (end 182.765 69.1) (width 0.2) (layer "F.Cu") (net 14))
 (segment (start 187.96 70.104) (end 187.96 68.836) (width 0.2) (layer "F.Cu") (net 14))
 (segment (start 182.765 69.1) (end 177.280001 69.1) (width 0.2) (layer "F.Cu") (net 14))
 (segment (start 187.96 68.836) (end 188.016 68.78) (width 0.2) (layer "F.Cu") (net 14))
 (via (at 183.515 69.85) (size 0.6) (drill 0.3) (layers "F.Cu" "B.Cu") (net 14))
 (via (at 187.96 70.104) (size 0.6) (drill 0.3) (layers "F.Cu" "B.Cu") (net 14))
 (segment (start 183.746 70.081) (end 187.937 70.081) (width 0.2) (layer "B.Cu") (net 14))
 (segment (start 183.515 69.85) (end 183.746 70.081) (width 0.2) (layer "B.Cu") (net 14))
 (segment (start 187.937 70.081) (end 187.96 70.104) (width 0.2) (layer "B.Cu") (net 14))
 (segment (start 177.280001 66.9) (end 181.61 66.9) (width 0.2) (layer "F.Cu") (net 15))
 (segment (start 186.016 70.310472) (end 185.645472 70.681) (width 0.2) (layer "F.Cu") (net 15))
 (segment (start 186.016 68.78) (end 186.016 70.310472) (width 0.2) (layer "F.Cu") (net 15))
 (via (at 181.61 66.9) (size 0.6) (drill 0.3) (layers "F.Cu" "B.Cu") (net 15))
 (via (at 185.645472 70.681) (size 0.6) (drill 0.3) (layers "F.Cu" "B.Cu") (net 15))
 (segment (start 181.61 69.215) (end 181.61 66.9) (width 0.2) (layer "B.Cu") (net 15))
 (segment (start 185.645472 70.681) (end 183.076 70.681) (width 0.2) (layer "B.Cu") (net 15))
 (segment (start 183.076 70.681) (end 181.61 69.215) (width 0.2) (layer "B.Cu") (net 15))
 (segment (start 175.524 72.4) (end 175.514 72.39) (width 0.2) (layer "F.Cu") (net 12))
 (segment (start 189.992 60.198) (end 189.992 61.856001) (width 0.2) (layer "F.Cu") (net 12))
 (segment (start 177.28 72.4) (end 175.524 72.4) (width 0.2) (layer "F.Cu") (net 12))
 (segment (start 189.992 61.856001) (end 190.015999 61.88) (width 0.2) (layer "F.Cu") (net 12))
 (via (at 175.514 72.39) (size 0.6) (drill 0.3) (layers "F.Cu" "B.Cu") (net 12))
 (via (at 189.992 60.198) (size 0.6) (drill 0.3) (layers "F.Cu" "B.Cu") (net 12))
 (segment (start 175.514 72.39) (end 175.514 69.847035) (width 0.2) (layer "B.Cu") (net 12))
 (segment (start 175.514 69.847035) (end 185.163035 60.198) (width 0.2) (layer "B.Cu") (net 12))
 (segment (start 185.163035 60.198) (end 189.992 60.198) (width 0.2) (layer "B.Cu") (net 12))
 (segment (start 179 64.7) (end 179.07 64.77) (width 0.2) (layer "F.Cu") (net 17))
 (segment (start 177.28 64.7) (end 179 64.7) (width 0.2) (layer "F.Cu") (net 17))
 (segment (start 189.016 59.5988) (end 189.016 61.880001) (width 0.2) (layer "F.Cu") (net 17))
 (segment (start 189.0152 59.598) (end 189.016 59.5988) (width 0.2) (layer "F.Cu") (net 17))
 (via (at 179.07 64.77) (size 0.6) (drill 0.3) (layers "F.Cu" "B.Cu") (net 17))
 (via (at 189.0152 59.598) (size 0.6) (drill 0.3) (layers "F.Cu" "B.Cu") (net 17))
 (segment (start 179.07 64.77) (end 184.242 59.598) (width 0.2) (layer "B.Cu") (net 17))
 (segment (start 184.242 59.598) (end 189.0152 59.598) (width 0.2) (layer "B.Cu") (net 17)))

